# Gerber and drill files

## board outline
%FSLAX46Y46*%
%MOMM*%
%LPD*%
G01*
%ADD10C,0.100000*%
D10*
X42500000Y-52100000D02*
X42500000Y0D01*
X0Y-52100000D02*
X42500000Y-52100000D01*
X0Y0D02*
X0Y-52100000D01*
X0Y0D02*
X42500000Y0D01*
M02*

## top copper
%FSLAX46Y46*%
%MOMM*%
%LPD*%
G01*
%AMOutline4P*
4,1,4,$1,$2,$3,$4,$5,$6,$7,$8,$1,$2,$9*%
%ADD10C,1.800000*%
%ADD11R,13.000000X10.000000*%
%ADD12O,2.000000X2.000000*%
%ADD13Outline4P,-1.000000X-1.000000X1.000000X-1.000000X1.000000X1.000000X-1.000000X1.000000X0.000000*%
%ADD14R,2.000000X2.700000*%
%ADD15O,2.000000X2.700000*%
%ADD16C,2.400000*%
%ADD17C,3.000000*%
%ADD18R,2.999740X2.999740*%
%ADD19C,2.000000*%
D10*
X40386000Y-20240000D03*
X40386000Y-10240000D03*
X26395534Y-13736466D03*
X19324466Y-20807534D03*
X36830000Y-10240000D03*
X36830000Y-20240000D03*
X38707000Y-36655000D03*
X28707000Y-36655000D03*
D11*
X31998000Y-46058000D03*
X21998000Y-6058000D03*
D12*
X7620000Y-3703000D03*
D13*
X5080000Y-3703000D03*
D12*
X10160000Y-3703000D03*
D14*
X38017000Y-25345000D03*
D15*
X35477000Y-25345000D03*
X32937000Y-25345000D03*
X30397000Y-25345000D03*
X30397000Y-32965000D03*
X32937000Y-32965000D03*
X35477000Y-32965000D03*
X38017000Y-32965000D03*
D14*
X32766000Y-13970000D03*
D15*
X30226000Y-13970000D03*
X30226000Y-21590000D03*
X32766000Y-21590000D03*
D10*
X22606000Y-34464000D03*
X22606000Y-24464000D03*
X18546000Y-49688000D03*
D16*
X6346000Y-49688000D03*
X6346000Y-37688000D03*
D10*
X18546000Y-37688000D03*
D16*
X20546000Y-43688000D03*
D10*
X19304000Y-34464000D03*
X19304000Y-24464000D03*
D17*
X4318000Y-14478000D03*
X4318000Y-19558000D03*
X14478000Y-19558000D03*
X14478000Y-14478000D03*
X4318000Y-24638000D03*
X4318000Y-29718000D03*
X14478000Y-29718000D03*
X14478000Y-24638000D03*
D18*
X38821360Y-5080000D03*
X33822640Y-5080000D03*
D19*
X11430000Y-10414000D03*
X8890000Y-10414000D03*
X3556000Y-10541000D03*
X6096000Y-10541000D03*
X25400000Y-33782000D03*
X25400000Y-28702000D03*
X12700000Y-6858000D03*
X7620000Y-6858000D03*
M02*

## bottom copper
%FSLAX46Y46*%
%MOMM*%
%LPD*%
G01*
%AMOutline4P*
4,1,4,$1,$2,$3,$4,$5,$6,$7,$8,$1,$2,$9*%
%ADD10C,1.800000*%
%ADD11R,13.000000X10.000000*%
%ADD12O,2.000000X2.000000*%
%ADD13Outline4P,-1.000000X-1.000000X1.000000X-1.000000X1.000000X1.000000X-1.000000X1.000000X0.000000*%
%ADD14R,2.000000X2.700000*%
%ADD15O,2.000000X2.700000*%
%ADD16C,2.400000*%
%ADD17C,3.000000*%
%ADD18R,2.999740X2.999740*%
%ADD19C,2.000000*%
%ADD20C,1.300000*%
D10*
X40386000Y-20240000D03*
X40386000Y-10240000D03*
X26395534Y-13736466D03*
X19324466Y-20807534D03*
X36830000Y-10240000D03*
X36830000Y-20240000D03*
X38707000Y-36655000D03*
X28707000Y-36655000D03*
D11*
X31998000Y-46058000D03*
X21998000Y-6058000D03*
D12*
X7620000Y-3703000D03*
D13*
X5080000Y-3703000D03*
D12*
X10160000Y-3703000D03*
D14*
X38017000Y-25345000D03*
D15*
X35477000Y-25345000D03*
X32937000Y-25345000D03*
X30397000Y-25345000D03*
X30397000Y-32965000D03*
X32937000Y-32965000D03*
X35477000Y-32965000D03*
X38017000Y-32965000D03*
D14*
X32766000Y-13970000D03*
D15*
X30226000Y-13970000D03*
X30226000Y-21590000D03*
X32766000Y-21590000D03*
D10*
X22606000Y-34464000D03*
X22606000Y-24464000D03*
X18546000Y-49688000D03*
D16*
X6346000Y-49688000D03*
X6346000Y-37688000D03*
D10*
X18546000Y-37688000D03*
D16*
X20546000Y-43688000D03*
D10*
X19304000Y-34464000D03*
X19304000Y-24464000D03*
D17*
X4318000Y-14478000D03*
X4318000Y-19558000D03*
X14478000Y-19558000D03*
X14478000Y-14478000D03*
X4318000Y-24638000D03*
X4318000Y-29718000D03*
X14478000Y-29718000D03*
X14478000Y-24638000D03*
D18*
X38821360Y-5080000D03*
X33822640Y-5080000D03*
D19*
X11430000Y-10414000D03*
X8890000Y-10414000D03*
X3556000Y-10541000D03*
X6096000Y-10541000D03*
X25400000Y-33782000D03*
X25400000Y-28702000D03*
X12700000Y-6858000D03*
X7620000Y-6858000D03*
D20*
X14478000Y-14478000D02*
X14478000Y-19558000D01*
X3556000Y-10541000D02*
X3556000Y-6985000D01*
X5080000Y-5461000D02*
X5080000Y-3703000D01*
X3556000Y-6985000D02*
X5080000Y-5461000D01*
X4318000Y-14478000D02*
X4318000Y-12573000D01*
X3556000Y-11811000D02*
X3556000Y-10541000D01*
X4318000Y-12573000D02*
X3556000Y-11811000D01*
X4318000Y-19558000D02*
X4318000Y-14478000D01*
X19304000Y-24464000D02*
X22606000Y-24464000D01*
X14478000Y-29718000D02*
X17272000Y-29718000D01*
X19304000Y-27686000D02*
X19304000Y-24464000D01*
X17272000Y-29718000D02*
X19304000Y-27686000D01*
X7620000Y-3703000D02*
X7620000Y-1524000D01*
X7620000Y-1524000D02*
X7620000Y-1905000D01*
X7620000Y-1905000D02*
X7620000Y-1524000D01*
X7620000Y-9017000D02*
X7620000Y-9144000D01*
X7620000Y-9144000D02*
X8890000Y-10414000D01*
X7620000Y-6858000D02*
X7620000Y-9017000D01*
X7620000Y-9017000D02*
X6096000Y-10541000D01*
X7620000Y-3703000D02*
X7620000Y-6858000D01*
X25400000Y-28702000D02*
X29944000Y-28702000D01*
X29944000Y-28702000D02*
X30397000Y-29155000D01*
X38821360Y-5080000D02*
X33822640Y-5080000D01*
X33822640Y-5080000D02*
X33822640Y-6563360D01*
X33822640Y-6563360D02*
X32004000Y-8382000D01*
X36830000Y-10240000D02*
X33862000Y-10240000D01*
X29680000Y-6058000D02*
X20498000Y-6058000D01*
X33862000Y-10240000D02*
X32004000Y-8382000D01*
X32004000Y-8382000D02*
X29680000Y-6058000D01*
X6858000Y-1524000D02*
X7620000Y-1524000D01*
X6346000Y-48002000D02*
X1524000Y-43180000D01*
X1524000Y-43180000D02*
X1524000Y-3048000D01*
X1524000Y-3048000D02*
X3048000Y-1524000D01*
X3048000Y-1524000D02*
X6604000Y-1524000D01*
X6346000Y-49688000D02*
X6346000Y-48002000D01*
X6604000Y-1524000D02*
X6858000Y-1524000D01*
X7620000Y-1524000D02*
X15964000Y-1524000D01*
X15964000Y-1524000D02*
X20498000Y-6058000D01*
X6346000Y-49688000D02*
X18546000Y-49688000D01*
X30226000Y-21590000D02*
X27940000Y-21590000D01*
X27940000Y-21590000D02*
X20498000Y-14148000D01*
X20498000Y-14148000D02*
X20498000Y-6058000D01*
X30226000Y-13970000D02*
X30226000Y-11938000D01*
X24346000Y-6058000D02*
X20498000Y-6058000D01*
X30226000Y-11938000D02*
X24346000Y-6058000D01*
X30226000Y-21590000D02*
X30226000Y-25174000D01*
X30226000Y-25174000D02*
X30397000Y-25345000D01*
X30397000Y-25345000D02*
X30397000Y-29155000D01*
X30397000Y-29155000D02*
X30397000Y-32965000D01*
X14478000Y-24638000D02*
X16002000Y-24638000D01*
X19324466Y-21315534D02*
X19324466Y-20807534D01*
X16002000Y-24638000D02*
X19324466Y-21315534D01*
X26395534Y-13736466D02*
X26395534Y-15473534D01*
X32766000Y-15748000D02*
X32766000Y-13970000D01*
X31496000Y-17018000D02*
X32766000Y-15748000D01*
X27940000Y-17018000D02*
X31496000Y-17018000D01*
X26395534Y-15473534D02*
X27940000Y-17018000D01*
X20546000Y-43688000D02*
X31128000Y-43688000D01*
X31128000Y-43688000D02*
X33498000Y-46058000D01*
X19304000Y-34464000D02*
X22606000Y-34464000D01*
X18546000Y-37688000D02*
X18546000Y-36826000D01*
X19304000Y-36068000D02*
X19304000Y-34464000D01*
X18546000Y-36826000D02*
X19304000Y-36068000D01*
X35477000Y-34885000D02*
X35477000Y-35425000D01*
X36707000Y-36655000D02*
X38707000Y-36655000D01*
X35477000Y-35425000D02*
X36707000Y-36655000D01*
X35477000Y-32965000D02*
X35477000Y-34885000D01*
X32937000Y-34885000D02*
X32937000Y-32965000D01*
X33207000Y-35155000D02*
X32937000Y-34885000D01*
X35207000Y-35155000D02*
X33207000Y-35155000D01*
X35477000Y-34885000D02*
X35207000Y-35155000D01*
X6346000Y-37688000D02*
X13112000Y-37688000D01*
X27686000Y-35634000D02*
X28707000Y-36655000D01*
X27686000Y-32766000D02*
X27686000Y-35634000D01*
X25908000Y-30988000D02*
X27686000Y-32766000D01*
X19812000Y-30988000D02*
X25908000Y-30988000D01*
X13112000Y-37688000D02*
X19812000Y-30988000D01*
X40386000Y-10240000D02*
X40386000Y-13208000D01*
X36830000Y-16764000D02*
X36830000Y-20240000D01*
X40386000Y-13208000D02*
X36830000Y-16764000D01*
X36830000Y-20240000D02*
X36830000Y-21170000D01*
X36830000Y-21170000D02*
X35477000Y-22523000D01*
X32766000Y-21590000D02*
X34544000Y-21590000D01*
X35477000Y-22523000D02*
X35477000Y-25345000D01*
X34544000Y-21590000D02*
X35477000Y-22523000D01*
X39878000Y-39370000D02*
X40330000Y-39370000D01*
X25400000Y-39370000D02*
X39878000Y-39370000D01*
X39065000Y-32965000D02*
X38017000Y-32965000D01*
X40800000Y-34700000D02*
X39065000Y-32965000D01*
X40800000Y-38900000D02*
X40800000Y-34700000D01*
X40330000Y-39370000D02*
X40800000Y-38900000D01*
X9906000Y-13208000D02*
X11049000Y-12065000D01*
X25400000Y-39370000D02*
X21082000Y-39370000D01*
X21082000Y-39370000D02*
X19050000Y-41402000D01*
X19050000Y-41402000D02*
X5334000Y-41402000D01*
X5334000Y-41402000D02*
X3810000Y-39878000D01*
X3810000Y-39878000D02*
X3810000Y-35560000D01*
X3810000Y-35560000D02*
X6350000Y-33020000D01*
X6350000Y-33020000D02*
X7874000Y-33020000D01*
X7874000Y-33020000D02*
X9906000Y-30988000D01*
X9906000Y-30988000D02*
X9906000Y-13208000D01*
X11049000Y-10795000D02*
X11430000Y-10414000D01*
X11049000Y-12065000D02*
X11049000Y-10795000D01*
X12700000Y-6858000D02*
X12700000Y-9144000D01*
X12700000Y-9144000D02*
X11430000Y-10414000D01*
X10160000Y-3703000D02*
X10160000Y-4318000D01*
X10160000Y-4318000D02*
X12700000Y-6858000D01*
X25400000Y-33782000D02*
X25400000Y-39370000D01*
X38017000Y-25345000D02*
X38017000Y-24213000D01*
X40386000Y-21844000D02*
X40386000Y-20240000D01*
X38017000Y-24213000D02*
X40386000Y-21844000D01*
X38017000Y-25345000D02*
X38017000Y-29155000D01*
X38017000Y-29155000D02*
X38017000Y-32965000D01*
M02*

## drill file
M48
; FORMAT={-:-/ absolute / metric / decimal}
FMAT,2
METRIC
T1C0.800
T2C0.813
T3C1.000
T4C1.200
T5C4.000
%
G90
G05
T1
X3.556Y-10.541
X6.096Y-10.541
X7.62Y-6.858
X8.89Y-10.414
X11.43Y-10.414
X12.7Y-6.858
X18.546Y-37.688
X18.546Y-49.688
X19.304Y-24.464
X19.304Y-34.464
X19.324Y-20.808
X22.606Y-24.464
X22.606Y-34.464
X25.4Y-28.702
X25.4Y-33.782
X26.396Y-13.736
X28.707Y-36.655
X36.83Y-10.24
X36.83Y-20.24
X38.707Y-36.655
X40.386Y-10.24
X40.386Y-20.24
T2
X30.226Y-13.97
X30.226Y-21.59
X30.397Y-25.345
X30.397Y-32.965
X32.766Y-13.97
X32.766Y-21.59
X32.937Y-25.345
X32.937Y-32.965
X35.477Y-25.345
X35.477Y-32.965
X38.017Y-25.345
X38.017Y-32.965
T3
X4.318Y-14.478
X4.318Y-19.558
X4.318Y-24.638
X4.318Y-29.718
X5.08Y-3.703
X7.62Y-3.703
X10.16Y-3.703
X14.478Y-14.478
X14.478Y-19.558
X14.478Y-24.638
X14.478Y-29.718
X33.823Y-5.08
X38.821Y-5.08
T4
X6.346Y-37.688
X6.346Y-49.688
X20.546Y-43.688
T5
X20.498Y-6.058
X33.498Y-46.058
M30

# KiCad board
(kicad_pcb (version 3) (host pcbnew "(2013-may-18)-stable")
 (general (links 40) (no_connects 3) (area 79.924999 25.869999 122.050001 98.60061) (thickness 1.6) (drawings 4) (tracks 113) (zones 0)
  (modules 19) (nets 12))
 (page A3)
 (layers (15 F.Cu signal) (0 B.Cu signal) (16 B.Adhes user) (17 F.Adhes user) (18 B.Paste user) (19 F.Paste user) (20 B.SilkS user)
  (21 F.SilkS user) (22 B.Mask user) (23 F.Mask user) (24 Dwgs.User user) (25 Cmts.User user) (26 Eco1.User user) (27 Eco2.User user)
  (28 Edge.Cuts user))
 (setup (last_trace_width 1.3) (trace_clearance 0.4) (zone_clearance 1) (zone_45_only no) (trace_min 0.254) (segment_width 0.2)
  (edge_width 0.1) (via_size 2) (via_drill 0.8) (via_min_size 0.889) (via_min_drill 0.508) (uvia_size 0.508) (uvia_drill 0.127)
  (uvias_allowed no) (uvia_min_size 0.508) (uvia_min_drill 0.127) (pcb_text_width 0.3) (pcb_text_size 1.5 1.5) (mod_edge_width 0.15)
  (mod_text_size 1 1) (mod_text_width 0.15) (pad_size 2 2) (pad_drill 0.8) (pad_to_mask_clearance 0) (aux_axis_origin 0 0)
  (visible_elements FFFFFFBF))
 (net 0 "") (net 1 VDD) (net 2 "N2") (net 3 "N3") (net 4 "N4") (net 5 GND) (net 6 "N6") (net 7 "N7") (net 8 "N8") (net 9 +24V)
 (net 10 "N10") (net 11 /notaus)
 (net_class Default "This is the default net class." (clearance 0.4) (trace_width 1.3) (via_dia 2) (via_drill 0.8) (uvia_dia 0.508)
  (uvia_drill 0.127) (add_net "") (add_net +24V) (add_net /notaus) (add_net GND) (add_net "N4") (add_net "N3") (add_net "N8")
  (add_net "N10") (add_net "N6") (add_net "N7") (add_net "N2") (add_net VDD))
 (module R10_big (layer F.Cu) (at 40.386 15.24 90) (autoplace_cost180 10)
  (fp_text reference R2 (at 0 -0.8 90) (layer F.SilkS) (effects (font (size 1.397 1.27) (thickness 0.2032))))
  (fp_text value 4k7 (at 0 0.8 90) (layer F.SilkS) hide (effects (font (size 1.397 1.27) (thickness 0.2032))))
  (pad 1 thru_hole circle (at -5 0 90) (size 1.8 1.8) (drill 0.8) (layers *.Cu *.Mask F.SilkS) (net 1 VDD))
  (pad 2 thru_hole circle (at 5 0 90) (size 1.8 1.8) (drill 0.8) (layers *.Cu *.Mask F.SilkS) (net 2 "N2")))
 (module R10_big (layer F.Cu) (at 22.86 17.272 225) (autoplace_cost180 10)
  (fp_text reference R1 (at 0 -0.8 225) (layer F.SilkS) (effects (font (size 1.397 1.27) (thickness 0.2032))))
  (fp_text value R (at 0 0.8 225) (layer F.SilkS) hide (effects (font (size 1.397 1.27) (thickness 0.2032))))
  (pad 1 thru_hole circle (at -5 0 225) (size 1.8 1.8) (drill 0.8) (layers *.Cu *.Mask F.SilkS) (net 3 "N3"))
  (pad 2 thru_hole circle (at 5 0 225) (size 1.8 1.8) (drill 0.8) (layers *.Cu *.Mask F.SilkS) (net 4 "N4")))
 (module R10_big (layer F.Cu) (at 36.83 15.24 270) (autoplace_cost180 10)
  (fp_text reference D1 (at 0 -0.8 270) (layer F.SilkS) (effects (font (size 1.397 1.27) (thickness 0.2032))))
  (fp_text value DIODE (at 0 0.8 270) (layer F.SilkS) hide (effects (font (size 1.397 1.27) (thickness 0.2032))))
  (pad 1 thru_hole circle (at -5 0 270) (size 1.8 1.8) (drill 0.8) (layers *.Cu *.Mask F.SilkS) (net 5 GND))
  (pad 2 thru_hole circle (at 5 0 270) (size 1.8 1.8) (drill 0.8) (layers *.Cu *.Mask F.SilkS) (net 2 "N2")))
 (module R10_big (layer F.Cu) (at 33.707 36.655 180) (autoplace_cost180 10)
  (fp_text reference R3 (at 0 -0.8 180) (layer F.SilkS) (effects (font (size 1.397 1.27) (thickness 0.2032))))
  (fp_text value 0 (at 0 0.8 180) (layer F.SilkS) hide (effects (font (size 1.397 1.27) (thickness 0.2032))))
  (pad 1 thru_hole circle (at -5 0 180) (size 1.8 1.8) (drill 0.8) (layers *.Cu *.Mask F.SilkS) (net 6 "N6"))
  (pad 2 thru_hole circle (at 5 0 180) (size 1.8 1.8) (drill 0.8) (layers *.Cu *.Mask F.SilkS) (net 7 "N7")))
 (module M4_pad (layer F.Cu) (at 33.498 46.058 180)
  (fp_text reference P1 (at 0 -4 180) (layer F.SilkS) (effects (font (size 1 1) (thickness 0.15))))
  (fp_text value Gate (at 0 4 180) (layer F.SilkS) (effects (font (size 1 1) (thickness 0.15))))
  (pad 1 thru_hole rect (at 0 0 180) (size 13 10) (drill 4 (offset 1.5 0)) (layers *.Cu *.Mask F.SilkS) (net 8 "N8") (clearance 1)))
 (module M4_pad (layer F.Cu) (at 20.498 6.058)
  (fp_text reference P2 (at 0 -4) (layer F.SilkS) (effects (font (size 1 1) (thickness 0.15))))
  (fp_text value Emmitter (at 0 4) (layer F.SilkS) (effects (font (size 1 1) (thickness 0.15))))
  (pad 1 thru_hole rect (at 0 0) (size 13 10) (drill 4 (offset 1.5 0)) (layers *.Cu *.Mask F.SilkS) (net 5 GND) (clearance 1)))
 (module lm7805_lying (layer F.Cu) (at 7.62 -14.097)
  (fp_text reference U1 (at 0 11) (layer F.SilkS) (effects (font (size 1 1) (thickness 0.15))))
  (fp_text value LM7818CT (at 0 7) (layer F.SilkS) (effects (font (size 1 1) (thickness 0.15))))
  (pad 2 thru_hole oval (at 0 17.8) (size 2 2) (drill 1) (layers *.Cu *.Mask F.SilkS) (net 5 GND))
  (pad 1 thru_hole trapezoid (at -2.54 17.8) (size 2 2) (drill 1) (layers *.Cu *.Mask F.SilkS) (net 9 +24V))
  (pad 3 thru_hole oval (at 2.54 17.8) (size 2 2) (drill 1) (layers *.Cu *.Mask F.SilkS) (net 1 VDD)))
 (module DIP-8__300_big (layer F.Cu) (at 34.207 29.155 180)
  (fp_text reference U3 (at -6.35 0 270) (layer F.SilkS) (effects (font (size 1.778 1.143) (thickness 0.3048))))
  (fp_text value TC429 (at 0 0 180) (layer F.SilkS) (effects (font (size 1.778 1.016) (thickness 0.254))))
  (pad 1 thru_hole rect (at -3.81 3.81 180) (size 2 2.7) (drill 0.8128) (layers *.Cu *.Mask F.SilkS) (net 1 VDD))
  (pad 2 thru_hole oval (at -1.27 3.81 180) (size 2 2.7) (drill 0.8128) (layers *.Cu *.Mask F.SilkS) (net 2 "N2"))
  (pad 3 thru_hole oval (at 1.27 3.81 180) (size 2 2.7) (drill 0.8128) (layers *.Cu *.Mask F.SilkS))
  (pad 4 thru_hole oval (at 3.81 3.81 180) (size 2 2.7) (drill 0.8128) (layers *.Cu *.Mask F.SilkS) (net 5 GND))
  (pad 5 thru_hole oval (at 3.81 -3.81 180) (size 2 2.7) (drill 0.8128) (layers *.Cu *.Mask F.SilkS) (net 5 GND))
  (pad 6 thru_hole oval (at 1.27 -3.81 180) (size 2 2.7) (drill 0.8128) (layers *.Cu *.Mask F.SilkS) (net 6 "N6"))
  (pad 7 thru_hole oval (at -1.27 -3.81 180) (size 2 2.7) (drill 0.8128) (layers *.Cu *.Mask F.SilkS) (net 6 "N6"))
  (pad 8 thru_hole oval (at -3.81 -3.81 180) (size 2 2.7) (drill 0.8128) (layers *.Cu *.Mask F.SilkS) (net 1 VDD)))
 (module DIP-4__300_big (layer F.Cu) (at 31.496 17.78 180)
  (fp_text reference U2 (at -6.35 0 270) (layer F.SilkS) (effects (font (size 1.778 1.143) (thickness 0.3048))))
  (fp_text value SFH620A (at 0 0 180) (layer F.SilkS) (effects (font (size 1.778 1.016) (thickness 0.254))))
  (pad 1 thru_hole rect (at -1.27 3.81 180) (size 2 2.7) (drill 0.8128) (layers *.Cu *.Mask F.SilkS) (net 3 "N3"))
  (pad 2 thru_hole oval (at 1.27 3.81 180) (size 2 2.7) (drill 0.8128) (layers *.Cu *.Mask F.SilkS) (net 5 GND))
  (pad 3 thru_hole oval (at 1.27 -3.81 180) (size 2 2.7) (drill 0.8128) (layers *.Cu *.Mask F.SilkS) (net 5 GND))
  (pad 4 thru_hole oval (at -1.27 -3.81 180) (size 2 2.7) (drill 0.8128) (layers *.Cu *.Mask F.SilkS) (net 2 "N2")))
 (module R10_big (layer F.Cu) (at 22.606 29.464 90) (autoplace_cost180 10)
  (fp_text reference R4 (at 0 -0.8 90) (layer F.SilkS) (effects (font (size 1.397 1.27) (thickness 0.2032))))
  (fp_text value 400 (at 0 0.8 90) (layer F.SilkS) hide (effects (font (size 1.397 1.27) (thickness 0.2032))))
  (pad 1 thru_hole circle (at -5 0 90) (size 1.8 1.8) (drill 0.8) (layers *.Cu *.Mask F.SilkS) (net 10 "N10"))
  (pad 2 thru_hole circle (at 5 0 90) (size 1.8 1.8) (drill 0.8) (layers *.Cu *.Mask F.SilkS) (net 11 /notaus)))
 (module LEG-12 (layer F.Cu) (at 12.446 43.688 180)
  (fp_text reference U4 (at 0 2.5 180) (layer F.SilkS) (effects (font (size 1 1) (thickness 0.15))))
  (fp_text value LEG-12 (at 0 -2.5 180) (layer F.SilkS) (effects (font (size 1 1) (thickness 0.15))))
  (pad 1 thru_hole circle (at -6.1 -6 180) (size 1.8 1.8) (drill 0.8) (layers *.Cu *.Mask F.SilkS) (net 5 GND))
  (pad 5 thru_hole circle (at 6.1 -6 180) (size 2.4 2.4) (drill 1.2) (layers *.Cu *.Mask F.SilkS) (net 5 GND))
  (pad 4 thru_hole circle (at 6.1 6 180) (size 2.4 2.4) (drill 1.2) (layers *.Cu *.Mask F.SilkS) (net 7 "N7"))
  (pad 2 thru_hole circle (at -6.1 6 180) (size 1.8 1.8) (drill 0.8) (layers *.Cu *.Mask F.SilkS) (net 10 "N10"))
  (pad 3 thru_hole circle (at -8.1 0 180) (size 2.4 2.4) (drill 1.2) (layers *.Cu *.Mask F.SilkS) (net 8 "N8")))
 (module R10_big (layer F.Cu) (at 19.304 29.464 90) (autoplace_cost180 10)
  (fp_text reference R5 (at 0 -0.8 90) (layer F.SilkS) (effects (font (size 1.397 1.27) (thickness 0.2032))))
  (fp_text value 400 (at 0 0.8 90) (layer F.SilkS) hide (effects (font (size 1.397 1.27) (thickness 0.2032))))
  (pad 1 thru_hole circle (at -5 0 90) (size 1.8 1.8) (drill 0.8) (layers *.Cu *.Mask F.SilkS) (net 10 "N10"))
  (pad 2 thru_hole circle (at 5 0 90) (size 1.8 1.8) (drill 0.8) (layers *.Cu *.Mask F.SilkS) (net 11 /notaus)))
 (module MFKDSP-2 (layer F.Cu) (at 9.398 17.018)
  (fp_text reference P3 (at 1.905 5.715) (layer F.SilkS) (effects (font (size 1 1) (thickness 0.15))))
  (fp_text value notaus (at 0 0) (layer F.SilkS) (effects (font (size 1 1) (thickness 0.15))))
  (pad 1 thru_hole circle (at -5.08 -2.54) (size 3 3) (drill 1) (layers *.Cu *.Mask F.SilkS) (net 9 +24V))
  (pad 2 thru_hole circle (at -5.08 2.54) (size 3 3) (drill 1) (layers *.Cu *.Mask F.SilkS) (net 9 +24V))
  (pad 2 thru_hole circle (at 5.08 2.54) (size 3 3) (drill 1) (layers *.Cu *.Mask F.SilkS) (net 9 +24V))
  (pad 1 thru_hole circle (at 5.08 -2.54) (size 3 3) (drill 1) (layers *.Cu *.Mask F.SilkS) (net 9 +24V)))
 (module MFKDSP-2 (layer F.Cu) (at 9.398 27.178)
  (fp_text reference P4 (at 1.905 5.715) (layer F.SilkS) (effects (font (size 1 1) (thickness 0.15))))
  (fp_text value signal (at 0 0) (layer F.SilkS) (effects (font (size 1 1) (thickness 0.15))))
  (pad 1 thru_hole circle (at -5.08 -2.54) (size 3 3) (drill 1) (layers *.Cu *.Mask F.SilkS) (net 4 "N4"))
  (pad 2 thru_hole circle (at -5.08 2.54) (size 3 3) (drill 1) (layers *.Cu *.Mask F.SilkS) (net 11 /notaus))
  (pad 2 thru_hole circle (at 5.08 2.54) (size 3 3) (drill 1) (layers *.Cu *.Mask F.SilkS) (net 11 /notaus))
  (pad 1 thru_hole circle (at 5.08 -2.54) (size 3 3) (drill 1) (layers *.Cu *.Mask F.SilkS) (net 4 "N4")))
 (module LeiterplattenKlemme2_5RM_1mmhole (layer F.Cu) (at 36.322 5.08)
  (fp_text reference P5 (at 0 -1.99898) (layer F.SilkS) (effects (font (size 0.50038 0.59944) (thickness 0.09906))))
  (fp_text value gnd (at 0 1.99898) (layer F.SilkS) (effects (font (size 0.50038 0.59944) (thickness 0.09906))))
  (pad 1 thru_hole rect (at 2.49936 0) (size 2.99974 2.99974) (drill 1) (layers *.Cu *.Mask F.SilkS) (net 5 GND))
  (pad 2 thru_hole rect (at -2.49936 0) (size 2.99974 2.99974) (drill 1) (layers *.Cu *.Mask F.SilkS) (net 5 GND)))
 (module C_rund (layer F.Cu) (at 10.16 10.414 180)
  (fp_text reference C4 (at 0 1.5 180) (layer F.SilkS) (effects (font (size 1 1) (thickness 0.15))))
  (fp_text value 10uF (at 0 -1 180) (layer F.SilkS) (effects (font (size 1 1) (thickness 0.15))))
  (pad 1 thru_hole circle (at -1.27 0 180) (size 2 2) (drill 0.8) (layers *.Cu *.Mask F.SilkS) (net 1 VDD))
  (pad 2 thru_hole circle (at 1.27 0 180) (size 2 2) (drill 0.8) (layers *.Cu *.Mask F.SilkS) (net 5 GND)))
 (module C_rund (layer F.Cu) (at 4.826 10.541)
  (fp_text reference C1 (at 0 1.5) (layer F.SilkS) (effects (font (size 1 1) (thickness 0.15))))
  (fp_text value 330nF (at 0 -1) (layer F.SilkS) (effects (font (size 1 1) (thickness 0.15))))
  (pad 1 thru_hole circle (at -1.27 0) (size 2 2) (drill 0.8) (layers *.Cu *.Mask F.SilkS) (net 9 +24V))
  (pad 2 thru_hole circle (at 1.27 0) (size 2 2) (drill 0.8) (layers *.Cu *.Mask F.SilkS) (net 5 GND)))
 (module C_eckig (layer F.Cu) (at 25.4 31.242 90)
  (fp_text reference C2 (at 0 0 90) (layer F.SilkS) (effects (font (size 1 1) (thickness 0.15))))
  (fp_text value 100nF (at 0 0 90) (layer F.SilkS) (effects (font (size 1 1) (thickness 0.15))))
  (pad 1 thru_hole circle (at -2.54 0 90) (size 2 2) (drill 0.8) (layers *.Cu *.Mask F.SilkS) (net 1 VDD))
  (pad 2 thru_hole circle (at 2.54 0 90) (size 2 2) (drill 0.8) (layers *.Cu *.Mask F.SilkS) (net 5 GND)))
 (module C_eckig (layer F.Cu) (at 10.16 6.858 180)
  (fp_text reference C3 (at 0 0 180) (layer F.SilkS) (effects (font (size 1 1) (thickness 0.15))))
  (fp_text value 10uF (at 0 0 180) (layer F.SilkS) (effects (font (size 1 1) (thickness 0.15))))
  (pad 1 thru_hole circle (at -2.54 0 180) (size 2 2) (drill 0.8) (layers *.Cu *.Mask F.SilkS) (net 1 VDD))
  (pad 2 thru_hole circle (at 2.54 0 180) (size 2 2) (drill 0.8) (layers *.Cu *.Mask F.SilkS) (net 5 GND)))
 (gr_line (start 42.5 52.1) (end 42.5 0) (angle 90) (layer Edge.Cuts) (width 0.1))
 (gr_line (start 0 52.1) (end 42.5 52.1) (angle 90) (layer Edge.Cuts) (width 0.1))
 (gr_line (start 0 0) (end 0 52.1) (angle 90) (layer Edge.Cuts) (width 0.1))
 (gr_line (start 0 0) (end 42.5 0) (angle 90) (layer Edge.Cuts) (width 0.1))
 (segment (start 14.478 14.478) (end 14.478 19.558) (width 1.3) (layer B.Cu) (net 9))
 (segment (start 3.556 10.541) (end 3.556 6.985) (width 1.3) (layer B.Cu) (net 9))
 (segment (start 5.08 5.461) (end 5.08 3.703) (width 1.3) (layer B.Cu) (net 9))
 (segment (start 3.556 6.985) (end 5.08 5.461) (width 1.3) (layer B.Cu) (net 9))
 (segment (start 4.318 14.478) (end 4.318 12.573) (width 1.3) (layer B.Cu) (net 9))
 (segment (start 3.556 11.811) (end 3.556 10.541) (width 1.3) (layer B.Cu) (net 9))
 (segment (start 4.318 12.573) (end 3.556 11.811) (width 1.3) (layer B.Cu) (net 9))
 (segment (start 4.318 19.558) (end 4.318 14.478) (width 1.3) (layer B.Cu) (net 9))
 (segment (start 19.304 24.464) (end 22.606 24.464) (width 1.3) (layer B.Cu) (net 11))
 (segment (start 14.478 29.718) (end 17.272 29.718) (width 1.3) (layer B.Cu) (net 11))
 (segment (start 19.304 27.686) (end 19.304 24.464) (width 1.3) (layer B.Cu) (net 11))
 (segment (start 17.272 29.718) (end 19.304 27.686) (width 1.3) (layer B.Cu) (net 11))
 (segment (start 7.62 3.703) (end 7.62 1.524) (width 1.3) (layer B.Cu) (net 5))
 (segment (start 7.62 1.524) (end 7.62 1.905) (width 1.3) (layer B.Cu) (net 5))
 (segment (start 7.62 1.905) (end 7.62 1.524) (width 1.3) (layer B.Cu) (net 5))
 (segment (start 7.62 9.017) (end 7.62 9.144) (width 1.3) (layer B.Cu) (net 5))
 (segment (start 7.62 9.144) (end 8.89 10.414) (width 1.3) (layer B.Cu) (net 5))
 (segment (start 7.62 6.858) (end 7.62 9.017) (width 1.3) (layer B.Cu) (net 5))
 (segment (start 7.62 9.017) (end 6.096 10.541) (width 1.3) (layer B.Cu) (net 5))
 (segment (start 7.62 3.703) (end 7.62 6.858) (width 1.3) (layer B.Cu) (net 5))
 (segment (start 25.4 28.702) (end 29.944 28.702) (width 1.3) (layer B.Cu) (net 5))
 (segment (start 29.944 28.702) (end 30.397 29.155) (width 1.3) (layer B.Cu) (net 5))
 (segment (start 38.82136 5.08) (end 33.82264 5.08) (width 1.3) (layer B.Cu) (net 5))
 (segment (start 33.82264 5.08) (end 33.82264 6.56336) (width 1.3) (layer B.Cu) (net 5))
 (segment (start 33.82264 6.56336) (end 32.004 8.382) (width 1.3) (layer B.Cu) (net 5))
 (segment (start 36.83 10.24) (end 33.862 10.24) (width 1.3) (layer B.Cu) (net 5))
 (segment (start 29.68 6.058) (end 20.498 6.058) (width 1.3) (layer B.Cu) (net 5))
 (segment (start 33.862 10.24) (end 32.004 8.382) (width 1.3) (layer B.Cu) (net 5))
 (segment (start 32.004 8.382) (end 29.68 6.058) (width 1.3) (layer B.Cu) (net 5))
 (segment (start 6.858 1.524) (end 7.62 1.524) (width 1.3) (layer B.Cu) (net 5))
 (segment (start 6.346 48.002) (end 1.524 43.18) (width 1.3) (layer B.Cu) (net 5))
 (segment (start 1.524 43.18) (end 1.524 3.048) (width 1.3) (layer B.Cu) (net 5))
 (segment (start 1.524 3.048) (end 3.048 1.524) (width 1.3) (layer B.Cu) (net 5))
 (segment (start 3.048 1.524) (end 6.604 1.524) (width 1.3) (layer B.Cu) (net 5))
 (segment (start 6.346 49.688) (end 6.346 48.002) (width 1.3) (layer B.Cu) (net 5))
 (segment (start 6.604 1.524) (end 6.858 1.524) (width 1.3) (layer B.Cu) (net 5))
 (segment (start 7.62 1.524) (end 15.964 1.524) (width 1.3) (layer B.Cu) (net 5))
 (segment (start 15.964 1.524) (end 20.498 6.058) (width 1.3) (layer B.Cu) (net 5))
 (segment (start 6.346 49.688) (end 18.546 49.688) (width 1.3) (layer B.Cu) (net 5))
 (segment (start 30.226 21.59) (end 27.94 21.59) (width 1.3) (layer B.Cu) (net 5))
 (segment (start 27.94 21.59) (end 20.498 14.148) (width 1.3) (layer B.Cu) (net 5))
 (segment (start 20.498 14.148) (end 20.498 6.058) (width 1.3) (layer B.Cu) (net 5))
 (segment (start 30.226 13.97) (end 30.226 11.938) (width 1.3) (layer B.Cu) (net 5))
 (segment (start 24.346 6.058) (end 20.498 6.058) (width 1.3) (layer B.Cu) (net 5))
 (segment (start 30.226 11.938) (end 24.346 6.058) (width 1.3) (layer B.Cu) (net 5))
 (segment (start 30.226 21.59) (end 30.226 25.174) (width 1.3) (layer B.Cu) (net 5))
 (segment (start 30.226 25.174) (end 30.397 25.345) (width 1.3) (layer B.Cu) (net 5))
 (segment (start 30.397 25.345) (end 30.397 29.155) (width 1.3) (layer B.Cu) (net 5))
 (segment (start 30.397 29.155) (end 30.397 32.965) (width 1.3) (layer B.Cu) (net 5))
 (segment (start 14.478 24.638) (end 16.002 24.638) (width 1.3) (layer B.Cu) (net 4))
 (segment (start 19.324466 21.315534) (end 19.324466 20.807534) (width 1.3) (layer B.Cu) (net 4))
 (segment (start 16.002 24.638) (end 19.324466 21.315534) (width 1.3) (layer B.Cu) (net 4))
 (segment (start 26.395534 13.736466) (end 26.395534 15.473534) (width 1.3) (layer B.Cu) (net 3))
 (segment (start 32.766 15.748) (end 32.766 13.97) (width 1.3) (layer B.Cu) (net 3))
 (segment (start 31.496 17.018) (end 32.766 15.748) (width 1.3) (layer B.Cu) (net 3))
 (segment (start 27.94 17.018) (end 31.496 17.018) (width 1.3) (layer B.Cu) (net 3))
 (segment (start 26.395534 15.473534) (end 27.94 17.018) (width 1.3) (layer B.Cu) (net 3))
 (segment (start 20.546 43.688) (end 31.128 43.688) (width 1.3) (layer B.Cu) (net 8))
 (segment (start 31.128 43.688) (end 33.498 46.058) (width 1.3) (layer B.Cu) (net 8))
 (segment (start 19.304 34.464) (end 22.606 34.464) (width 1.3) (layer B.Cu) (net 10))
 (segment (start 18.546 37.688) (end 18.546 36.826) (width 1.3) (layer B.Cu) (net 10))
 (segment (start 19.304 36.068) (end 19.304 34.464) (width 1.3) (layer B.Cu) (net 10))
 (segment (start 18.546 36.826) (end 19.304 36.068) (width 1.3) (layer B.Cu) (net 10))
 (segment (start 35.477 34.885) (end 35.477 35.425) (width 1.3) (layer B.Cu) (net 6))
 (segment (start 36.707 36.655) (end 38.707 36.655) (width 1.3) (layer B.Cu) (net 6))
 (segment (start 35.477 35.425) (end 36.707 36.655) (width 1.3) (layer B.Cu) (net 6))
 (segment (start 35.477 32.965) (end 35.477 34.885) (width 1.3) (layer B.Cu) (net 6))
 (segment (start 32.937 34.885) (end 32.937 32.965) (width 1.3) (layer B.Cu) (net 6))
 (segment (start 33.207 35.155) (end 32.937 34.885) (width 1.3) (layer B.Cu) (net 6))
 (segment (start 35.207 35.155) (end 33.207 35.155) (width 1.3) (layer B.Cu) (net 6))
 (segment (start 35.477 34.885) (end 35.207 35.155) (width 1.3) (layer B.Cu) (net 6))
 (segment (start 6.346 37.688) (end 13.112 37.688) (width 1.3) (layer B.Cu) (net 7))
 (segment (start 27.686 35.634) (end 28.707 36.655) (width 1.3) (layer B.Cu) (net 7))
 (segment (start 27.686 32.766) (end 27.686 35.634) (width 1.3) (layer B.Cu) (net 7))
 (segment (start 25.908 30.988) (end 27.686 32.766) (width 1.3) (layer B.Cu) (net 7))
 (segment (start 19.812 30.988) (end 25.908 30.988) (width 1.3) (layer B.Cu) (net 7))
 (segment (start 13.112 37.688) (end 19.812 30.988) (width 1.3) (layer B.Cu) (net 7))
 (segment (start 40.386 10.24) (end 40.386 13.208) (width 1.3) (layer B.Cu) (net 2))
 (segment (start 36.83 16.764) (end 36.83 20.24) (width 1.3) (layer B.Cu) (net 2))
 (segment (start 40.386 13.208) (end 36.83 16.764) (width 1.3) (layer B.Cu) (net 2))
 (segment (start 36.83 20.24) (end 36.83 21.17) (width 1.3) (layer B.Cu) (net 2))
 (segment (start 36.83 21.17) (end 35.477 22.523) (width 1.3) (layer B.Cu) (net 2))
 (segment (start 32.766 21.59) (end 34.544 21.59) (width 1.3) (layer B.Cu) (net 2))
 (segment (start 35.477 22.523) (end 35.477 25.345) (width 1.3) (layer B.Cu) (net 2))
 (segment (start 34.544 21.59) (end 35.477 22.523) (width 1.3) (layer B.Cu) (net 2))
 (segment (start 39.878 39.37) (end 40.33 39.37) (width 1.3) (layer B.Cu) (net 1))
 (segment (start 25.4 39.37) (end 39.878 39.37) (width 1.3) (layer B.Cu) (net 1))
 (segment (start 39.065 32.965) (end 38.017 32.965) (width 1.3) (layer B.Cu) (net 1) (status 800000))
 (segment (start 40.8 34.7) (end 39.065 32.965) (width 1.3) (layer B.Cu) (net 1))
 (segment (start 40.8 38.9) (end 40.8 34.7) (width 1.3) (layer B.Cu) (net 1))
 (segment (start 40.33 39.37) (end 40.8 38.9) (width 1.3) (layer B.Cu) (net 1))
 (segment (start 9.906 13.208) (end 11.049 12.065) (width 1.3) (layer B.Cu) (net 1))
 (segment (start 25.4 39.37) (end 21.082 39.37) (width 1.3) (layer B.Cu) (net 1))
 (segment (start 21.082 39.37) (end 19.05 41.402) (width 1.3) (layer B.Cu) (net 1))
 (segment (start 19.05 41.402) (end 5.334 41.402) (width 1.3) (layer B.Cu) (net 1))
 (segment (start 5.334 41.402) (end 3.81 39.878) (width 1.3) (layer B.Cu) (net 1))
 (segment (start 3.81 39.878) (end 3.81 35.56) (width 1.3) (layer B.Cu) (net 1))
 (segment (start 3.81 35.56) (end 6.35 33.02) (width 1.3) (layer B.Cu) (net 1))
 (segment (start 6.35 33.02) (end 7.874 33.02) (width 1.3) (layer B.Cu) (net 1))
 (segment (start 7.874 33.02) (end 9.906 30.988) (width 1.3) (layer B.Cu) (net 1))
 (segment (start 9.906 30.988) (end 9.906 13.208) (width 1.3) (layer B.Cu) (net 1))
 (segment (start 11.049 10.795) (end 11.43 10.414) (width 1.3) (layer B.Cu) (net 1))
 (segment (start 11.049 12.065) (end 11.049 10.795) (width 1.3) (layer B.Cu) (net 1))
 (segment (start 12.7 6.858) (end 12.7 9.144) (width 1.3) (layer B.Cu) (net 1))
 (segment (start 12.7 9.144) (end 11.43 10.414) (width 1.3) (layer B.Cu) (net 1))
 (segment (start 10.16 3.703) (end 10.16 4.318) (width 1.3) (layer B.Cu) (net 1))
 (segment (start 10.16 4.318) (end 12.7 6.858) (width 1.3) (layer B.Cu) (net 1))
 (segment (start 25.4 33.782) (end 25.4 39.37) (width 1.3) (layer B.Cu) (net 1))
 (segment (start 38.017 25.345) (end 38.017 24.213) (width 1.3) (layer B.Cu) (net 1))
 (segment (start 40.386 21.844) (end 40.386 20.24) (width 1.3) (layer B.Cu) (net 1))
 (segment (start 38.017 24.213) (end 40.386 21.844) (width 1.3) (layer B.Cu) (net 1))
 (segment (start 38.017 25.345) (end 38.017 29.155) (width 1.3) (layer B.Cu) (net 1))
 (segment (start 38.017 29.155) (end 38.017 32.965) (width 1.3) (layer B.Cu) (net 1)))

